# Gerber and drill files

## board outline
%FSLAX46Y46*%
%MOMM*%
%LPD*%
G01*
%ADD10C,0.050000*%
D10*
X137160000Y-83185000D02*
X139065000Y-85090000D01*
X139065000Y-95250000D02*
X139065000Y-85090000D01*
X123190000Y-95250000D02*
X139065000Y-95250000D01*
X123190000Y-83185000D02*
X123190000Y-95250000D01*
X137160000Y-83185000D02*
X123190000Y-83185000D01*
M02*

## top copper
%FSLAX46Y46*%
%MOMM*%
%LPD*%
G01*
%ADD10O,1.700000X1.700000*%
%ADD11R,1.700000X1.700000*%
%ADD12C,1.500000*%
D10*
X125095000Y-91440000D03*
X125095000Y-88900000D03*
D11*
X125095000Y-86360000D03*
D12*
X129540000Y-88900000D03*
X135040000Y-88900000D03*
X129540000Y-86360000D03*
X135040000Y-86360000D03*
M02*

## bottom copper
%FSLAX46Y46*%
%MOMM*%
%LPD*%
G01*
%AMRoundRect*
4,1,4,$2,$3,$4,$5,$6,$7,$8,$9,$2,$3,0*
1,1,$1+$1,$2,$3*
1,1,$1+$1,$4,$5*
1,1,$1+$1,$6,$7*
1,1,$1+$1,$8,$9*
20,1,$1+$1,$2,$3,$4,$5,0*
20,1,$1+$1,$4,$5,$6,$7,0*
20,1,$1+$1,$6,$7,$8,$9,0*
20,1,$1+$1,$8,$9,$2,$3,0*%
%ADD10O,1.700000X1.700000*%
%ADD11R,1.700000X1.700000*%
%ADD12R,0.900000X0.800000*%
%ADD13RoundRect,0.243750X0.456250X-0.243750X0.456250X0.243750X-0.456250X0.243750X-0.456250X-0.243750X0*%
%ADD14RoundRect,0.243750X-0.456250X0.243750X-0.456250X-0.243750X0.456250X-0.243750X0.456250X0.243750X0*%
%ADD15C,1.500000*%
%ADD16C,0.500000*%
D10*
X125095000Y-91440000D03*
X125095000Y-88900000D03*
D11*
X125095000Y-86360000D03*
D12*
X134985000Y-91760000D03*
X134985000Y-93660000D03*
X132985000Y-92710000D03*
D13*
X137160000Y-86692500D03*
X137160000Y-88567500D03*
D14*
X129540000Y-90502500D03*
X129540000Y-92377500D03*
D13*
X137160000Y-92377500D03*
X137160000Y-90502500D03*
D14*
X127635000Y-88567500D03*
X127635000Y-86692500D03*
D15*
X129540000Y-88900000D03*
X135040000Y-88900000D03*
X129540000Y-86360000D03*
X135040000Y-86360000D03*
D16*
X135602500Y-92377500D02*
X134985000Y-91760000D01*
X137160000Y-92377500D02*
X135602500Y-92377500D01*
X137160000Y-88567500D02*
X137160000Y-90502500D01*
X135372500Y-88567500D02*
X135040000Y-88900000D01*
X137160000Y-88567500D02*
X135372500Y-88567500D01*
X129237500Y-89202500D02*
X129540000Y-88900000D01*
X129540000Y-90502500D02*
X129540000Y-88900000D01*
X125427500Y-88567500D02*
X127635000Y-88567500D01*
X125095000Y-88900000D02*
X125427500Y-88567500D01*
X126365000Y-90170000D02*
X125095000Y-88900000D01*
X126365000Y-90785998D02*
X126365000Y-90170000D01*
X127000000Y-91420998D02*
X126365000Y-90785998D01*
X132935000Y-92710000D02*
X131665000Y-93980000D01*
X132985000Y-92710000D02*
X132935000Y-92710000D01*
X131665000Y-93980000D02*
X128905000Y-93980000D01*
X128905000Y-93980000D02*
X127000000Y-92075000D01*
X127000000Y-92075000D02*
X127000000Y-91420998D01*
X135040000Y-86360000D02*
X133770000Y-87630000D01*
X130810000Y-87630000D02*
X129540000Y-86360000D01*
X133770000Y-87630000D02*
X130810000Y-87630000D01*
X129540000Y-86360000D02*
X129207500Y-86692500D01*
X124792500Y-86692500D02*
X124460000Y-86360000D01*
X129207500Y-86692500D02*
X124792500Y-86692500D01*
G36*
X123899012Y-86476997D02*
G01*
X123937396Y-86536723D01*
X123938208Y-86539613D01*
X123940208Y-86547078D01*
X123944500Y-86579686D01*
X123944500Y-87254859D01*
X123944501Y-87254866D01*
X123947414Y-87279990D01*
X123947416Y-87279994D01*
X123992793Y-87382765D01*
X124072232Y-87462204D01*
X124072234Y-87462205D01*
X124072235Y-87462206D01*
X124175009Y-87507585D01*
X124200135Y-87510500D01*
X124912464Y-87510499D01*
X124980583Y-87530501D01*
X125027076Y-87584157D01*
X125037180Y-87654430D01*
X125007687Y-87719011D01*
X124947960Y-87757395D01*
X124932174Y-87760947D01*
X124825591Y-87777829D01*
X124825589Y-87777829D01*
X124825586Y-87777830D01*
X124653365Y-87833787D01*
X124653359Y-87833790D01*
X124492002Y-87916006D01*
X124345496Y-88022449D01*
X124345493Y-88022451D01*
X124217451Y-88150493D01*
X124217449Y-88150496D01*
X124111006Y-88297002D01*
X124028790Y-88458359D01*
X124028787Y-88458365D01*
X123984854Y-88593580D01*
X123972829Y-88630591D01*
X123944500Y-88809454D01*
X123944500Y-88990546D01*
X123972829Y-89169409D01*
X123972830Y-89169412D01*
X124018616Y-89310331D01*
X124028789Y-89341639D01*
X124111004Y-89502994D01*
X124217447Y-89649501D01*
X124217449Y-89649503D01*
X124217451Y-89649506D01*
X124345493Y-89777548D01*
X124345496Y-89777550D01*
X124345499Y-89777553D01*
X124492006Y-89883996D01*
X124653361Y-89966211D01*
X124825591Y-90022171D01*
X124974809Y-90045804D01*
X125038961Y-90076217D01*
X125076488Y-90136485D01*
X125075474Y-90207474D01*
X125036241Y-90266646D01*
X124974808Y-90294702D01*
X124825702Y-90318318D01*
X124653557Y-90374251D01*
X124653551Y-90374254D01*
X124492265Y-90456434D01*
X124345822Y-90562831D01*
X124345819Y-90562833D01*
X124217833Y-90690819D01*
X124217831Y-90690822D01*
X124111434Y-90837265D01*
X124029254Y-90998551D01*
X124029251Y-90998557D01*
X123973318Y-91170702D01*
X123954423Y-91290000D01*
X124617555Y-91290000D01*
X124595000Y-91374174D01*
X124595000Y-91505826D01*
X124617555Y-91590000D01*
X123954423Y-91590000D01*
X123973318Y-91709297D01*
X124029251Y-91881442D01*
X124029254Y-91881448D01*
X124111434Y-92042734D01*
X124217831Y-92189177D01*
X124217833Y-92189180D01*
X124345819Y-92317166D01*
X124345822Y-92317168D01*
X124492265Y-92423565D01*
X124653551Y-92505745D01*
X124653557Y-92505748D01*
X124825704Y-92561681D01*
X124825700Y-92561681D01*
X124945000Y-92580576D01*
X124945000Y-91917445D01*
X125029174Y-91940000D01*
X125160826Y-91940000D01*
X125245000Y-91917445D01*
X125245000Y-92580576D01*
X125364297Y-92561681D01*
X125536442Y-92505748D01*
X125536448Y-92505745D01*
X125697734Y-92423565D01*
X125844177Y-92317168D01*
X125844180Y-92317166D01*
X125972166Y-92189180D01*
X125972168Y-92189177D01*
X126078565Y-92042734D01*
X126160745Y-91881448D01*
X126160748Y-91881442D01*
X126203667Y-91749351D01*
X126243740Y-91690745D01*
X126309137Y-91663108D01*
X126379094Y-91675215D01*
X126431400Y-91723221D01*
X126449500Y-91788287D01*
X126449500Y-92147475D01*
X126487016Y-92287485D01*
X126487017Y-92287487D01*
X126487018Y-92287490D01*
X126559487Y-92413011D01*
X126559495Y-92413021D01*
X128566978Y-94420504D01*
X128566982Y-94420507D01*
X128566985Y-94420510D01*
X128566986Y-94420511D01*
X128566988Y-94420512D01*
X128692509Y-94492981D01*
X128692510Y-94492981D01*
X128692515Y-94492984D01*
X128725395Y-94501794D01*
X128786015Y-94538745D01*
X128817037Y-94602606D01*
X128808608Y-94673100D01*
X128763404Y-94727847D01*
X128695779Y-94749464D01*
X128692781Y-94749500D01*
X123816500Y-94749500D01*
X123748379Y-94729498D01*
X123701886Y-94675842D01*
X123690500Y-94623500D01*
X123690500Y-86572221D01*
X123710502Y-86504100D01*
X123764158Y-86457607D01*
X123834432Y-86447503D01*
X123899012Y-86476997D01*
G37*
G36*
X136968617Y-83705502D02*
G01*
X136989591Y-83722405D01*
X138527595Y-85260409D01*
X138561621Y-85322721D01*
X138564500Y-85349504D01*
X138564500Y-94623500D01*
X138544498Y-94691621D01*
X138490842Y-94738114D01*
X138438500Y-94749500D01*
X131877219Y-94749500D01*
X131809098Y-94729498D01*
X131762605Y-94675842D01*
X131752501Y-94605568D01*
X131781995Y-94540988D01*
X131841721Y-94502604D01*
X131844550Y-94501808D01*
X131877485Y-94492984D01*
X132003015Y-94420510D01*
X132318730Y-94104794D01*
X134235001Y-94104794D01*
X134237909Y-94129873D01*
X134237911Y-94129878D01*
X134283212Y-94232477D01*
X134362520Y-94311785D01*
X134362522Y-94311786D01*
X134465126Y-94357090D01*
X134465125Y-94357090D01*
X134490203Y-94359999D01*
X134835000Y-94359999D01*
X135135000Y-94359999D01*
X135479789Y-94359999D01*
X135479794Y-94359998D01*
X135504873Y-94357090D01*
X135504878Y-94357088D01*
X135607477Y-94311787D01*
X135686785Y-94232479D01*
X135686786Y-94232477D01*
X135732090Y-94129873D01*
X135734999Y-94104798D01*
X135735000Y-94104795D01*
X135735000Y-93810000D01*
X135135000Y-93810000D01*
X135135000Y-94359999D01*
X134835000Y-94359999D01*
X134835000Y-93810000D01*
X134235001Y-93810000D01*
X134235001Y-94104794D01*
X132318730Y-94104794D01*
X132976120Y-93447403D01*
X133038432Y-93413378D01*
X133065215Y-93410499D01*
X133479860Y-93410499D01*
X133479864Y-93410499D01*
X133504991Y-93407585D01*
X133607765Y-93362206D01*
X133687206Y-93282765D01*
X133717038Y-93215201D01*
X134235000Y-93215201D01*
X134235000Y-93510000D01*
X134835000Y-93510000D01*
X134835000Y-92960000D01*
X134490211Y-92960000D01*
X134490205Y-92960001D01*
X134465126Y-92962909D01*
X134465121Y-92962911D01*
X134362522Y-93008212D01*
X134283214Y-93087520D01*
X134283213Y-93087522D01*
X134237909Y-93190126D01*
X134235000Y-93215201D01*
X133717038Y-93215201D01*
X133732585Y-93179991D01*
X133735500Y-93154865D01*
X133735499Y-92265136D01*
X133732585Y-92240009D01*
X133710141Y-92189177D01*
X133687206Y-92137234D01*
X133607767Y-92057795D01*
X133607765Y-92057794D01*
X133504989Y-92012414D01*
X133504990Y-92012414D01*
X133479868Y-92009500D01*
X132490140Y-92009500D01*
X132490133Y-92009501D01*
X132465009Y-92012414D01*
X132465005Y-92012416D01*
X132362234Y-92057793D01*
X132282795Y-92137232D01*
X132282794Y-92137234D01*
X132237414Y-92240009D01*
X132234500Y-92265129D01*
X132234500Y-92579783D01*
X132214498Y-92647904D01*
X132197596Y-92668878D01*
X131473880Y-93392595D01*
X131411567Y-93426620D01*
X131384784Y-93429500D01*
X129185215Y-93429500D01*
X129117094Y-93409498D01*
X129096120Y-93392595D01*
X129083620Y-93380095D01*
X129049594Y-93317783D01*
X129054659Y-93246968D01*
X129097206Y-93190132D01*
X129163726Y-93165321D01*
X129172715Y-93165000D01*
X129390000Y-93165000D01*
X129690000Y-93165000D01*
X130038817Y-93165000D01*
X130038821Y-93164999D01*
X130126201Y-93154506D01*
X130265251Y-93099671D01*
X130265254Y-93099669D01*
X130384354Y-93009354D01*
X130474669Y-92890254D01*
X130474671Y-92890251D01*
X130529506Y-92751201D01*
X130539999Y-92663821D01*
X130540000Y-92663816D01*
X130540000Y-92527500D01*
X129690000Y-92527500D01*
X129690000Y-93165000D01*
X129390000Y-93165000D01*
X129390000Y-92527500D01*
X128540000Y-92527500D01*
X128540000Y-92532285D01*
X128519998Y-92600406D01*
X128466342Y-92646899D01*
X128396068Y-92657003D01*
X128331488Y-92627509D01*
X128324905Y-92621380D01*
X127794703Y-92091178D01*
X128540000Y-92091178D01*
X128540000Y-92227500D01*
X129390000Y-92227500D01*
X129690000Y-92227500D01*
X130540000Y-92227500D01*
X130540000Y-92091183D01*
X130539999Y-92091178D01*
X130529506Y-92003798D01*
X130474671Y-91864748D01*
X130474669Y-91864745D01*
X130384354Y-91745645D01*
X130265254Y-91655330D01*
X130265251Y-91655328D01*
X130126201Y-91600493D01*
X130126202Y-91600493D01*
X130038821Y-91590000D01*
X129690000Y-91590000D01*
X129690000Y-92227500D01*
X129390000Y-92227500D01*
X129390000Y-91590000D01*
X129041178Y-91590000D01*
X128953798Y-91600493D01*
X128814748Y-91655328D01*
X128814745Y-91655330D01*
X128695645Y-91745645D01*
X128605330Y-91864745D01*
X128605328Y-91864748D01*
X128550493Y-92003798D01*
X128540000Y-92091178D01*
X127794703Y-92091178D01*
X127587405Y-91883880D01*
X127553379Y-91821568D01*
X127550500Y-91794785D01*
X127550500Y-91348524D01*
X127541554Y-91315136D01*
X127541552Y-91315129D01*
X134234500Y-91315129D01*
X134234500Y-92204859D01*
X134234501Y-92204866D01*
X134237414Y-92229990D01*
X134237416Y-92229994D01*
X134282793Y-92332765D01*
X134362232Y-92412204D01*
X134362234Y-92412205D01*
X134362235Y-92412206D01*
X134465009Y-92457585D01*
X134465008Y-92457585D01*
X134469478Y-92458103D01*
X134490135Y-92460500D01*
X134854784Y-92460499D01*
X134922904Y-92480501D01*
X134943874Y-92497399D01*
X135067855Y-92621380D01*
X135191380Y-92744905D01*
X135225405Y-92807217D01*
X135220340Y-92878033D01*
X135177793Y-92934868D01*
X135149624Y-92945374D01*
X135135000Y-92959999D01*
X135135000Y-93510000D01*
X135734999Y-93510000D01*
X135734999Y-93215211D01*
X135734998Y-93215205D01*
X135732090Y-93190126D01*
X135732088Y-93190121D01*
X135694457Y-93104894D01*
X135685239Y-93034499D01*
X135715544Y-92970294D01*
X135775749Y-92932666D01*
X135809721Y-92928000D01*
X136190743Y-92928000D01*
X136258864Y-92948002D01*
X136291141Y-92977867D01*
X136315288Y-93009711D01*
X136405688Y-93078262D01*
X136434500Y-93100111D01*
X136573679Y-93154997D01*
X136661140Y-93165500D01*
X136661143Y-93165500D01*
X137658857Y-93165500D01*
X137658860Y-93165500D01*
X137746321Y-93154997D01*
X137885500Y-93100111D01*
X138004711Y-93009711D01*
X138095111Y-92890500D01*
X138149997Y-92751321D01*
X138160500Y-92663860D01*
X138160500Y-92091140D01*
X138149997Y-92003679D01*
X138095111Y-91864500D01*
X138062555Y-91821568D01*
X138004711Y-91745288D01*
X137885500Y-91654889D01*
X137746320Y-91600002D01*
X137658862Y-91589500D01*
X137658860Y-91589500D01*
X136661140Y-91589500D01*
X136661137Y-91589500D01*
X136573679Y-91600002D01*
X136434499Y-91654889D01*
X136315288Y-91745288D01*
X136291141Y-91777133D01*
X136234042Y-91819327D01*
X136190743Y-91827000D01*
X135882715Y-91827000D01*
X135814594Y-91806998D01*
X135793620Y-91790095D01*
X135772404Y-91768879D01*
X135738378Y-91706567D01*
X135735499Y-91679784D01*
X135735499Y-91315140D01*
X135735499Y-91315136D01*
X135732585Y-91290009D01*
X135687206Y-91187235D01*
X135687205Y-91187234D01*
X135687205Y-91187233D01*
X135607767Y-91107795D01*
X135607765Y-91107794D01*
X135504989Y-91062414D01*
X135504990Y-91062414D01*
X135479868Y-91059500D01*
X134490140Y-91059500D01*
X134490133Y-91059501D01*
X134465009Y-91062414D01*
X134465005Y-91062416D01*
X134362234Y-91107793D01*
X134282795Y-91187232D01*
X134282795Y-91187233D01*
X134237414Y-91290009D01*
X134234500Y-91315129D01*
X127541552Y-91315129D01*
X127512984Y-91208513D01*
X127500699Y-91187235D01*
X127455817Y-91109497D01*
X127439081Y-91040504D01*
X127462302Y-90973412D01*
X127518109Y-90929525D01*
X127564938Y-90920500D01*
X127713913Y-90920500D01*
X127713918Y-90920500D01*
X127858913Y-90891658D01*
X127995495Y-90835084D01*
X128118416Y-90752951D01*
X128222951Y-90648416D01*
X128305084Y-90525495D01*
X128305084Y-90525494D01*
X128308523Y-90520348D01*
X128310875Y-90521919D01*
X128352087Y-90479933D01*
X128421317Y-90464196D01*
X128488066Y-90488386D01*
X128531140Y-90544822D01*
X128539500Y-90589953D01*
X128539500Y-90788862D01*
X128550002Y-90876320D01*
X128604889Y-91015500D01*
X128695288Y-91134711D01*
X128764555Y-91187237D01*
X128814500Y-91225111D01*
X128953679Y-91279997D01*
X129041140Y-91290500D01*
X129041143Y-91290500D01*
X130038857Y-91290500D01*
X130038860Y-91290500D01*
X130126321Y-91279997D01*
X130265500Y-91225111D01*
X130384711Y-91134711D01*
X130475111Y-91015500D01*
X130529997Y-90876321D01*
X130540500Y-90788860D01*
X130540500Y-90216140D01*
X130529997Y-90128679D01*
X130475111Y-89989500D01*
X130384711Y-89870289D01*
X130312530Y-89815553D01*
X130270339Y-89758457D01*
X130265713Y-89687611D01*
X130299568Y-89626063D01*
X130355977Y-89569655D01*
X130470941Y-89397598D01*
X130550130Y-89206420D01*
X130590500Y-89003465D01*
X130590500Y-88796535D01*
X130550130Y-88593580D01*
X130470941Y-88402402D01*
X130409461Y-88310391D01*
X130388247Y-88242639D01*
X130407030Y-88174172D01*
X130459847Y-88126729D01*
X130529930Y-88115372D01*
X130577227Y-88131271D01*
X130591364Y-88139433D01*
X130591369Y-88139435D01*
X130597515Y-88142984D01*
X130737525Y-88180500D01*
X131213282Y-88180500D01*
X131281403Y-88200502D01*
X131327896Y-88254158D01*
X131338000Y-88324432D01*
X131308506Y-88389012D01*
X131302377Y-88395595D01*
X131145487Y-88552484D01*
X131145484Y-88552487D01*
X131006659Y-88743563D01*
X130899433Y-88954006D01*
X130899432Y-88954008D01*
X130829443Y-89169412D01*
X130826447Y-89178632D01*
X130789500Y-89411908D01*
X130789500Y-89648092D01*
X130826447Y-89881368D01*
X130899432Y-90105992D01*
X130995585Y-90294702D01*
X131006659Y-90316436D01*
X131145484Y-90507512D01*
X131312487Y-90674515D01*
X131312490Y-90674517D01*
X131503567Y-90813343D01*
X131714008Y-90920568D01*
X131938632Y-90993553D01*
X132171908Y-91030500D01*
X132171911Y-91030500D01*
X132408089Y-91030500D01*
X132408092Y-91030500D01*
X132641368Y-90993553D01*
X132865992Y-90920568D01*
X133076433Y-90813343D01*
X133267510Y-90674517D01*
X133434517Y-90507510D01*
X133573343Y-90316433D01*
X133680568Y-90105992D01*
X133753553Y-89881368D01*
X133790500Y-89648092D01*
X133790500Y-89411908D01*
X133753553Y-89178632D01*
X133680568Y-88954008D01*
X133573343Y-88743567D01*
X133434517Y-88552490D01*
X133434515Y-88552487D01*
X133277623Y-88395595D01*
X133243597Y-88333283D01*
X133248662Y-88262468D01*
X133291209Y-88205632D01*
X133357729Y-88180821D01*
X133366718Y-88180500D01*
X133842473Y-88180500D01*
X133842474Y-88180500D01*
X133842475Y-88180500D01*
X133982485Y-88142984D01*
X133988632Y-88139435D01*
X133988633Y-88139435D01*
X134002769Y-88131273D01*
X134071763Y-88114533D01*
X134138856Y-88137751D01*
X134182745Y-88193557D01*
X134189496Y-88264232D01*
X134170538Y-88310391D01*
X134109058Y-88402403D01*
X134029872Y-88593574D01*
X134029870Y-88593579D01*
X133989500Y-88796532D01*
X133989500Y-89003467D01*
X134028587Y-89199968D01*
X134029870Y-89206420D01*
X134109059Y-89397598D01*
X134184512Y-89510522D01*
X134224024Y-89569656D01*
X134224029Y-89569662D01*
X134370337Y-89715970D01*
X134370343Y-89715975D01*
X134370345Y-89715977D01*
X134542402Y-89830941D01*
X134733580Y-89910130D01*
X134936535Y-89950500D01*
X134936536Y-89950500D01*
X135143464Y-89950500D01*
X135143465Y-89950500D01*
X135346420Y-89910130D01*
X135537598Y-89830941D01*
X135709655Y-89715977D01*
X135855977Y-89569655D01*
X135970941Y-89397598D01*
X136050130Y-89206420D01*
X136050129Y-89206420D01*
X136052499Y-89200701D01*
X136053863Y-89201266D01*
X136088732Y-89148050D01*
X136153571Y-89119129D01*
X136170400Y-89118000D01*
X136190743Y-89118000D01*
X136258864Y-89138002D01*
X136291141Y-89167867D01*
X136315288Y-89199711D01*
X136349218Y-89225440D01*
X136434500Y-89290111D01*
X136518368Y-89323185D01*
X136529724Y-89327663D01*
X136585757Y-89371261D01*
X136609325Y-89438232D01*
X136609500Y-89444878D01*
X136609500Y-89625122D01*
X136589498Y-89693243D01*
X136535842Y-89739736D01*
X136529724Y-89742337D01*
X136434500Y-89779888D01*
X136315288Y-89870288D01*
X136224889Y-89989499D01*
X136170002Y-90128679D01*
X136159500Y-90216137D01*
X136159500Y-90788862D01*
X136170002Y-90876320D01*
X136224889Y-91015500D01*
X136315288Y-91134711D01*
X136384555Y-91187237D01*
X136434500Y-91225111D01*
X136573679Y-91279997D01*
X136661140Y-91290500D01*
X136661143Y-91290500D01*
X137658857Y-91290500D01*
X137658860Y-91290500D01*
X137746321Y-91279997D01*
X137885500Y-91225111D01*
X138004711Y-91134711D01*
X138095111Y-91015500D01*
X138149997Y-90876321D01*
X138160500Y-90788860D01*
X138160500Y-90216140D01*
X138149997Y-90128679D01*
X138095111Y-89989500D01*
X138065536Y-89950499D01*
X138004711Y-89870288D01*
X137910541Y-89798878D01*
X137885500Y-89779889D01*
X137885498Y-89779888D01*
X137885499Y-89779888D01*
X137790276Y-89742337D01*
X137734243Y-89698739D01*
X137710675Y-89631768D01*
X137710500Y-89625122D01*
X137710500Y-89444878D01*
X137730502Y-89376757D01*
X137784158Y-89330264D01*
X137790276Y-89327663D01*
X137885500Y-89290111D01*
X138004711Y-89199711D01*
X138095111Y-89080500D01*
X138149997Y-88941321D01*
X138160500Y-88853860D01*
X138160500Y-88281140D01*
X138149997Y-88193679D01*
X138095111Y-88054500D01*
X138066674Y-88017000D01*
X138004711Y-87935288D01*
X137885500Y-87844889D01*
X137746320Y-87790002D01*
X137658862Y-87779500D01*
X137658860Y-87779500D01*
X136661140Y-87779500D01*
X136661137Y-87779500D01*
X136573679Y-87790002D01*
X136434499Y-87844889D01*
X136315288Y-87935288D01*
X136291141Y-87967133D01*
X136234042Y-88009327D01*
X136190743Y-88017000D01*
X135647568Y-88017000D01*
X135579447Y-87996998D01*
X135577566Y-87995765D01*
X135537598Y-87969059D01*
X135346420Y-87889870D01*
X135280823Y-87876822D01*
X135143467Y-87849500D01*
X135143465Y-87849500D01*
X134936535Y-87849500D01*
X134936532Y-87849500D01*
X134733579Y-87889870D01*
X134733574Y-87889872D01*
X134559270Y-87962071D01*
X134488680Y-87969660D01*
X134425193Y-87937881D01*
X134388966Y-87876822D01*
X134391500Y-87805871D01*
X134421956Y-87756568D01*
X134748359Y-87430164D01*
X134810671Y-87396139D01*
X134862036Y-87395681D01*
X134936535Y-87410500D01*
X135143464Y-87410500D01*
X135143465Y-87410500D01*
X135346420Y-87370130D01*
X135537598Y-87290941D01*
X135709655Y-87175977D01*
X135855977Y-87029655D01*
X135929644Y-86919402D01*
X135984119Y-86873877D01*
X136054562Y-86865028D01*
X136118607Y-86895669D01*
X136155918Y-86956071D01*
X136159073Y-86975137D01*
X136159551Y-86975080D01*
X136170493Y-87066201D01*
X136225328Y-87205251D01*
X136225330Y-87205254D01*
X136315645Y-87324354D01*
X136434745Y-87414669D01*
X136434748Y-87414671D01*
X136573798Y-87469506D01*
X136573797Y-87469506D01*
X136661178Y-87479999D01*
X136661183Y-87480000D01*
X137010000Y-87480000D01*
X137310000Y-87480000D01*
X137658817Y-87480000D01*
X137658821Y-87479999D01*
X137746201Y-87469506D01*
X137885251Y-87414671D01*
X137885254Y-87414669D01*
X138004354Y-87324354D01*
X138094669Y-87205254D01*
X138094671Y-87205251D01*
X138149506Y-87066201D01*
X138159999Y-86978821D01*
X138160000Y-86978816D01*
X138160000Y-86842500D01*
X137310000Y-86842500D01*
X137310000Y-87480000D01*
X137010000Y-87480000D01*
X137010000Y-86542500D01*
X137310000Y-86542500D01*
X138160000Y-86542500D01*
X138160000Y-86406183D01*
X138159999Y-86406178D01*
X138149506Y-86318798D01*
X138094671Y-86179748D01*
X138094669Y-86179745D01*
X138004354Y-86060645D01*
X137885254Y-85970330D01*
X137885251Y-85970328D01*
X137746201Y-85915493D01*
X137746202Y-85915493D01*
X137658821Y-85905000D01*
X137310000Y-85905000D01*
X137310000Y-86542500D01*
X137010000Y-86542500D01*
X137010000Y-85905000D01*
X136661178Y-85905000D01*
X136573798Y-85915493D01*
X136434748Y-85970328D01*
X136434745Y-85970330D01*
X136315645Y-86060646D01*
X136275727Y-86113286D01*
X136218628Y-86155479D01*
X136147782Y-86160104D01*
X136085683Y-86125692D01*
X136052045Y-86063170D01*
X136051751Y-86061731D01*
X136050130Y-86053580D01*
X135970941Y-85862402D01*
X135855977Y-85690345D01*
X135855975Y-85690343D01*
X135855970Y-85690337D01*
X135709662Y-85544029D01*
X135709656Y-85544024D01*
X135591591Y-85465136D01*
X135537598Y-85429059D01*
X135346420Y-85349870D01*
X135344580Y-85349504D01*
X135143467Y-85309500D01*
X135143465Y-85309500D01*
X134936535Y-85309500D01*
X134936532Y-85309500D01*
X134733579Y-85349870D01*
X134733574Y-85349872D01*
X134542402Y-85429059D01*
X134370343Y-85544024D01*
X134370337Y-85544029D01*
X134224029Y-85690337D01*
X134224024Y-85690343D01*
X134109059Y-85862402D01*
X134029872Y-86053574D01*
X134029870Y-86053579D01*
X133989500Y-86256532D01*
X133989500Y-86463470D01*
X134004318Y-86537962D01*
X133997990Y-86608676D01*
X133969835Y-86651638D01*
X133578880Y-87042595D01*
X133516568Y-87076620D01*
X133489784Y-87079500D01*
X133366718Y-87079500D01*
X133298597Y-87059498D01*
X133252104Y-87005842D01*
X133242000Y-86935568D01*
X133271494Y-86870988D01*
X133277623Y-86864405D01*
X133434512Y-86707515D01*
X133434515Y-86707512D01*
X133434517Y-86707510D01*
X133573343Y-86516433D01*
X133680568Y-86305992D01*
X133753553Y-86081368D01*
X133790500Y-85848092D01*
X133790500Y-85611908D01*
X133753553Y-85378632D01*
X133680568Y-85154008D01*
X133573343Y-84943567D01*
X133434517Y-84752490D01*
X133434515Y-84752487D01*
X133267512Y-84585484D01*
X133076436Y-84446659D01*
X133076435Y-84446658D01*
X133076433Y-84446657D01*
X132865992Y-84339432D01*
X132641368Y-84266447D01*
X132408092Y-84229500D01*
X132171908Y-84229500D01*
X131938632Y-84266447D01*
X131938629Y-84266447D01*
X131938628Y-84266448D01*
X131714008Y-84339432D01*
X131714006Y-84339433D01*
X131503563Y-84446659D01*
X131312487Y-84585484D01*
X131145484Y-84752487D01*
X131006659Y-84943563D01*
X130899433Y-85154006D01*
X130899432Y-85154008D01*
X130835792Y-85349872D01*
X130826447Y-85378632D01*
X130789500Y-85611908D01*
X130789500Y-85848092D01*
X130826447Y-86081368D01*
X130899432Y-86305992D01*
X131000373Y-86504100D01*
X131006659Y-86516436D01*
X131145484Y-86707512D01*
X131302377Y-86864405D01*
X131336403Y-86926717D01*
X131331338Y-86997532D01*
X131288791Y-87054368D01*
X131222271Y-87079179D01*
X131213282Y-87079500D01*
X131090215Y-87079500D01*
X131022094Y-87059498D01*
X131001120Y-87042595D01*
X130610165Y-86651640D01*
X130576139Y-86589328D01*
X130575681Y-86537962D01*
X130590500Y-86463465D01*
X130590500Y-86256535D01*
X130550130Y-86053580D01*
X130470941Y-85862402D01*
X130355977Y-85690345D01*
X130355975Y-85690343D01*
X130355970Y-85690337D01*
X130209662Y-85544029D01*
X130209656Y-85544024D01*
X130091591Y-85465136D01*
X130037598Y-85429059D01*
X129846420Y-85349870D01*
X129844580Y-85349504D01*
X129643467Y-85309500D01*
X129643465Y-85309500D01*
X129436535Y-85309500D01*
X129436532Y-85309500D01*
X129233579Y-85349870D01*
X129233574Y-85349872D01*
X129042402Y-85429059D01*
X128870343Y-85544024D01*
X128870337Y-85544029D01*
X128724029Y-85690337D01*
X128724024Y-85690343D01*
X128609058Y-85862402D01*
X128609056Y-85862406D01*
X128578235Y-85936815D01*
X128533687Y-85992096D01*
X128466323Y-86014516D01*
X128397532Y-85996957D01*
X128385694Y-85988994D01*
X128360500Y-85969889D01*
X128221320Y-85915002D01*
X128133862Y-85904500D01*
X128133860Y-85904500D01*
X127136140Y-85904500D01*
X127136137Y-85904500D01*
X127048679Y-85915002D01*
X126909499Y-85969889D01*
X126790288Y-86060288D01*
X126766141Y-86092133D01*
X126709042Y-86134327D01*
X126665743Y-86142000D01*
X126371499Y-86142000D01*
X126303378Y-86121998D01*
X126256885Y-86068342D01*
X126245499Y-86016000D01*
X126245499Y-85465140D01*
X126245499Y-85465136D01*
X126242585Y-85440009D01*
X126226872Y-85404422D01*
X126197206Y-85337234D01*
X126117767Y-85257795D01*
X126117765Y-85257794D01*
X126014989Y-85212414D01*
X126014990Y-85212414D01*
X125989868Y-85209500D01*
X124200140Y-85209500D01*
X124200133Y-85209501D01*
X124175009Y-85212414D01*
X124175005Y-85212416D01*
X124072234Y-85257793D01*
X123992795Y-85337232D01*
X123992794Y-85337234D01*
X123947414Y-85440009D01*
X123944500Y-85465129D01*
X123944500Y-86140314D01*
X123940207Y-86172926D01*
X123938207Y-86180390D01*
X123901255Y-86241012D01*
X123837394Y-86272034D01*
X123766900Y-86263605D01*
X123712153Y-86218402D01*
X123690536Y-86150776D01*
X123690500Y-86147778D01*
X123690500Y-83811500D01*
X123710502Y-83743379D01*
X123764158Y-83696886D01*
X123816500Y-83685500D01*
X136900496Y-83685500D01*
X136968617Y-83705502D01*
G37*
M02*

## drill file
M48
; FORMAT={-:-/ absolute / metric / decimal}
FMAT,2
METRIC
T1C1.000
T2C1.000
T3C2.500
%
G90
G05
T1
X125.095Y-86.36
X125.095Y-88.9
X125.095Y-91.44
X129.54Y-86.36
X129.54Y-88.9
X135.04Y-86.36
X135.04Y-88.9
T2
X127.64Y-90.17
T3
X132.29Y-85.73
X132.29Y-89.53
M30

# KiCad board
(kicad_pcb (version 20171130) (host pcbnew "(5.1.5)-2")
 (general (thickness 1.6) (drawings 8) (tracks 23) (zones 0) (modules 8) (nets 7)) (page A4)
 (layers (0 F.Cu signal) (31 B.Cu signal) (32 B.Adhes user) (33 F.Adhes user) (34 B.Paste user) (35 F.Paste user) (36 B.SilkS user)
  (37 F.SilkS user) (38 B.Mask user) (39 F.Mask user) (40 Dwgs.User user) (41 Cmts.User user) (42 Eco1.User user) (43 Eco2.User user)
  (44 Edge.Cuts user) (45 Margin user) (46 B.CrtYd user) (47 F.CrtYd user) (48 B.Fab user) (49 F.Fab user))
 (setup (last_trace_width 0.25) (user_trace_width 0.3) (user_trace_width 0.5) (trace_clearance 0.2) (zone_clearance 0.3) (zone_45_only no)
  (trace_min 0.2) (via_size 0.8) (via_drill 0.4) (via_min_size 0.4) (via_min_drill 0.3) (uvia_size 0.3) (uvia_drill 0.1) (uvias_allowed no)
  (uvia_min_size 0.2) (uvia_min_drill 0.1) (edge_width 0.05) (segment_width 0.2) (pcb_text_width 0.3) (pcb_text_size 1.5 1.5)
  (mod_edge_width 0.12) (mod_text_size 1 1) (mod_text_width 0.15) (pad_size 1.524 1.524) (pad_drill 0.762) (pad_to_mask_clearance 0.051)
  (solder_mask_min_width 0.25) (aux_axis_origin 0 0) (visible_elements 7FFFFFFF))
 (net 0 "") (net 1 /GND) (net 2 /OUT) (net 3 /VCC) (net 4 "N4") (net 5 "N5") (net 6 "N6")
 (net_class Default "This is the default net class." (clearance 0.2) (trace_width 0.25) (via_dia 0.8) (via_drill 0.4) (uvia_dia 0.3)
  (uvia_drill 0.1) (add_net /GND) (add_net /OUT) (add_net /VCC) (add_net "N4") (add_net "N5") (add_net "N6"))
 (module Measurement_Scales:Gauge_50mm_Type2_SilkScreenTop (layer F.Cu) (at 123.19 95.25)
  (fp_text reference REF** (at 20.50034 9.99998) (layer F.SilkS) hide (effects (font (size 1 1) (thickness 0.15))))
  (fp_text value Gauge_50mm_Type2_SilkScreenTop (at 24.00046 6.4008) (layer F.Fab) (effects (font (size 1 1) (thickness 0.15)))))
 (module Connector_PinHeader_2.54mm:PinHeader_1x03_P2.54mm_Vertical (layer F.Cu) (at 125.095 86.36)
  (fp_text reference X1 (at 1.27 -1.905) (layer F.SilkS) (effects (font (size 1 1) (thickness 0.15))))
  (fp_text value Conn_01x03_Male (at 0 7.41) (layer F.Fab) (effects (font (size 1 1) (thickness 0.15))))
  (pad 3 thru_hole oval (at 0 5.08) (size 1.7 1.7) (drill 1) (layers *.Cu *.Mask) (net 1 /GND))
  (pad 2 thru_hole oval (at 0 2.54) (size 1.7 1.7) (drill 1) (layers *.Cu *.Mask) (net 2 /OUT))
  (pad 1 thru_hole rect (at 0 0) (size 1.7 1.7) (drill 1) (layers *.Cu *.Mask) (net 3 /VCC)))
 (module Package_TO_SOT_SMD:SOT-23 (layer B.Cu) (at 133.985 92.71 180)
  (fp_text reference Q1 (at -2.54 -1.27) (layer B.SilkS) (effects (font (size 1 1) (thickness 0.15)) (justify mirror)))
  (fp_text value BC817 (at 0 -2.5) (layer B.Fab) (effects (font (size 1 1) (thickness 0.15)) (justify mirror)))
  (pad 1 smd rect (at -1 0.95 180) (size 0.9 0.8) (layers B.Cu B.Paste B.Mask) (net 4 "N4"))
  (pad 2 smd rect (at -1 -0.95 180) (size 0.9 0.8) (layers B.Cu B.Paste B.Mask) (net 1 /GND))
  (pad 3 smd rect (at 1 0 180) (size 0.9 0.8) (layers B.Cu B.Paste B.Mask) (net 2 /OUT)))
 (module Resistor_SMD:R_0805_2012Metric (layer B.Cu) (at 137.16 87.63 90)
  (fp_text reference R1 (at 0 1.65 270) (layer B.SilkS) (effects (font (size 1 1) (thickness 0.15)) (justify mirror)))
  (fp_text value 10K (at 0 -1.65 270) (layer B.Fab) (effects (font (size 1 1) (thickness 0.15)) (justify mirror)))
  (pad 2 smd roundrect (at 0.9375 0 90) (size 0.975 1.4) (layers B.Cu B.Paste B.Mask) (roundrect_rratio 0.25) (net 1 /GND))
  (pad 1 smd roundrect (at -0.9375 0 90) (size 0.975 1.4) (layers B.Cu B.Paste B.Mask) (roundrect_rratio 0.25) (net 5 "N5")))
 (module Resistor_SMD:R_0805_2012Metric (layer B.Cu) (at 129.54 91.44 270)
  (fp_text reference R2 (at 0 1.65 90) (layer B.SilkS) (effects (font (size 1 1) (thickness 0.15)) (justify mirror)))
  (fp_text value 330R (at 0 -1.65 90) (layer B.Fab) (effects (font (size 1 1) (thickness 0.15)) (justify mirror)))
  (pad 1 smd roundrect (at -0.9375 0 270) (size 0.975 1.4) (layers B.Cu B.Paste B.Mask) (roundrect_rratio 0.25) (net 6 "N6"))
  (pad 2 smd roundrect (at 0.9375 0 270) (size 0.975 1.4) (layers B.Cu B.Paste B.Mask) (roundrect_rratio 0.25) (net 1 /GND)))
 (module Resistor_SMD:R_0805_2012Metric (layer B.Cu) (at 137.16 91.44 90)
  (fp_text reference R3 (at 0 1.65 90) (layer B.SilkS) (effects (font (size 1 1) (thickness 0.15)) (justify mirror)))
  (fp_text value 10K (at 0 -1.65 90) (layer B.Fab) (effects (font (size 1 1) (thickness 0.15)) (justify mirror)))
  (pad 1 smd roundrect (at -0.9375 0 90) (size 0.975 1.4) (layers B.Cu B.Paste B.Mask) (roundrect_rratio 0.25) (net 4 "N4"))
  (pad 2 smd roundrect (at 0.9375 0 90) (size 0.975 1.4) (layers B.Cu B.Paste B.Mask) (roundrect_rratio 0.25) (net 5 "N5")))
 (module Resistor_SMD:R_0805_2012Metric (layer B.Cu) (at 127.635 87.63 270)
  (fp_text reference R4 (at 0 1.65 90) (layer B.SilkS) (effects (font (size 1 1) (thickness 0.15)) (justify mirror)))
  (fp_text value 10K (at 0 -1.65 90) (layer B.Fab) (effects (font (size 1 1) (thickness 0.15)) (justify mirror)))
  (pad 2 smd roundrect (at 0.9375 0 270) (size 0.975 1.4) (layers B.Cu B.Paste B.Mask) (roundrect_rratio 0.25) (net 2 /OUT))
  (pad 1 smd roundrect (at -0.9375 0 270) (size 0.975 1.4) (layers B.Cu B.Paste B.Mask) (roundrect_rratio 0.25) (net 3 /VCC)))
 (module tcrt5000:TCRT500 (layer F.Cu) (at 132.29 87.63)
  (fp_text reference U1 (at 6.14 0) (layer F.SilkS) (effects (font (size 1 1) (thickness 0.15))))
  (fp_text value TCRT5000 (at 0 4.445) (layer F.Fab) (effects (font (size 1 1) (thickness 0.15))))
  (pad "" np_thru_hole circle (at 0 -1.9) (size 2.5 2.5) (drill 2.5) (layers *.Cu *.Mask))
  (pad "" np_thru_hole circle (at 0 1.9) (size 2.5 2.5) (drill 2.5) (layers *.Cu *.Mask))
  (pad 3 thru_hole circle (at -2.75 1.27) (size 1.5 1.5) (drill 1) (layers *.Cu *.Mask) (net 6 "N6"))
  (pad 4 thru_hole circle (at 2.75 1.27) (size 1.5 1.5) (drill 1) (layers *.Cu *.Mask) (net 5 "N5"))
  (pad 1 thru_hole circle (at -2.75 -1.27) (size 1.5 1.5) (drill 1) (layers *.Cu *.Mask) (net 3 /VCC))
  (pad 2 thru_hole circle (at 2.75 -1.27) (size 1.5 1.5) (drill 1) (layers *.Cu *.Mask) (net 3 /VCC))
  (pad "" np_thru_hole circle (at -4.65 2.54) (size 1 1) (drill 1) (layers *.Cu *.Mask)))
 (gr_line (start 137.16 83.185) (end 139.065 85.09) (layer Edge.Cuts) (width 0.05))
 (gr_line (start 139.065 95.25) (end 139.065 85.09) (layer Edge.Cuts) (width 0.05))
 (gr_line (start 123.19 95.25) (end 139.065 95.25) (layer Edge.Cuts) (width 0.05))
 (gr_line (start 123.19 83.185) (end 123.19 95.25) (layer Edge.Cuts) (width 0.05))
 (gr_line (start 137.16 83.185) (end 123.19 83.185) (layer Edge.Cuts) (width 0.05))
 (segment (start 135.6025 92.3775) (end 134.985 91.76) (width 0.5) (layer B.Cu) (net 4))
 (segment (start 137.16 92.3775) (end 135.6025 92.3775) (width 0.5) (layer B.Cu) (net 4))
 (segment (start 137.16 88.5675) (end 137.16 90.5025) (width 0.5) (layer B.Cu) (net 5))
 (segment (start 135.3725 88.5675) (end 135.04 88.9) (width 0.5) (layer B.Cu) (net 5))
 (segment (start 137.16 88.5675) (end 135.3725 88.5675) (width 0.5) (layer B.Cu) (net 5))
 (segment (start 129.2375 89.2025) (end 129.54 88.9) (width 0.5) (layer B.Cu) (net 6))
 (segment (start 129.54 90.5025) (end 129.54 88.9) (width 0.5) (layer B.Cu) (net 6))
 (segment (start 125.4275 88.5675) (end 127.635 88.5675) (width 0.5) (layer B.Cu) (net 2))
 (segment (start 125.095 88.9) (end 125.4275 88.5675) (width 0.5) (layer B.Cu) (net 2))
 (segment (start 126.365 90.17) (end 125.095 88.9) (width 0.5) (layer B.Cu) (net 2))
 (segment (start 126.365 90.785998) (end 126.365 90.17) (width 0.5) (layer B.Cu) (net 2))
 (segment (start 127 91.420998) (end 126.365 90.785998) (width 0.5) (layer B.Cu) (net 2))
 (segment (start 132.935 92.71) (end 131.665 93.98) (width 0.5) (layer B.Cu) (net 2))
 (segment (start 132.985 92.71) (end 132.935 92.71) (width 0.5) (layer B.Cu) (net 2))
 (segment (start 131.665 93.98) (end 128.905 93.98) (width 0.5) (layer B.Cu) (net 2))
 (segment (start 128.905 93.98) (end 127 92.075) (width 0.5) (layer B.Cu) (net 2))
 (segment (start 127 92.075) (end 127 91.420998) (width 0.5) (layer B.Cu) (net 2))
 (segment (start 135.04 86.36) (end 133.77 87.63) (width 0.5) (layer B.Cu) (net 3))
 (segment (start 130.81 87.63) (end 129.54 86.36) (width 0.5) (layer B.Cu) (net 3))
 (segment (start 133.77 87.63) (end 130.81 87.63) (width 0.5) (layer B.Cu) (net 3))
 (segment (start 129.54 86.36) (end 129.2075 86.6925) (width 0.5) (layer B.Cu) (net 3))
 (segment (start 124.7925 86.6925) (end 124.46 86.36) (width 0.5) (layer B.Cu) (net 3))
 (segment (start 129.2075 86.6925) (end 124.7925 86.6925) (width 0.5) (layer B.Cu) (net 3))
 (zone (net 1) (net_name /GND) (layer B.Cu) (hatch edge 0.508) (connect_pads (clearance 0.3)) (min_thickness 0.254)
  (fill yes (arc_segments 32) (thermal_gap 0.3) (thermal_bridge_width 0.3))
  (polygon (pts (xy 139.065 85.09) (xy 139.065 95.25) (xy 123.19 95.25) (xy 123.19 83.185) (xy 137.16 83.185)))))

